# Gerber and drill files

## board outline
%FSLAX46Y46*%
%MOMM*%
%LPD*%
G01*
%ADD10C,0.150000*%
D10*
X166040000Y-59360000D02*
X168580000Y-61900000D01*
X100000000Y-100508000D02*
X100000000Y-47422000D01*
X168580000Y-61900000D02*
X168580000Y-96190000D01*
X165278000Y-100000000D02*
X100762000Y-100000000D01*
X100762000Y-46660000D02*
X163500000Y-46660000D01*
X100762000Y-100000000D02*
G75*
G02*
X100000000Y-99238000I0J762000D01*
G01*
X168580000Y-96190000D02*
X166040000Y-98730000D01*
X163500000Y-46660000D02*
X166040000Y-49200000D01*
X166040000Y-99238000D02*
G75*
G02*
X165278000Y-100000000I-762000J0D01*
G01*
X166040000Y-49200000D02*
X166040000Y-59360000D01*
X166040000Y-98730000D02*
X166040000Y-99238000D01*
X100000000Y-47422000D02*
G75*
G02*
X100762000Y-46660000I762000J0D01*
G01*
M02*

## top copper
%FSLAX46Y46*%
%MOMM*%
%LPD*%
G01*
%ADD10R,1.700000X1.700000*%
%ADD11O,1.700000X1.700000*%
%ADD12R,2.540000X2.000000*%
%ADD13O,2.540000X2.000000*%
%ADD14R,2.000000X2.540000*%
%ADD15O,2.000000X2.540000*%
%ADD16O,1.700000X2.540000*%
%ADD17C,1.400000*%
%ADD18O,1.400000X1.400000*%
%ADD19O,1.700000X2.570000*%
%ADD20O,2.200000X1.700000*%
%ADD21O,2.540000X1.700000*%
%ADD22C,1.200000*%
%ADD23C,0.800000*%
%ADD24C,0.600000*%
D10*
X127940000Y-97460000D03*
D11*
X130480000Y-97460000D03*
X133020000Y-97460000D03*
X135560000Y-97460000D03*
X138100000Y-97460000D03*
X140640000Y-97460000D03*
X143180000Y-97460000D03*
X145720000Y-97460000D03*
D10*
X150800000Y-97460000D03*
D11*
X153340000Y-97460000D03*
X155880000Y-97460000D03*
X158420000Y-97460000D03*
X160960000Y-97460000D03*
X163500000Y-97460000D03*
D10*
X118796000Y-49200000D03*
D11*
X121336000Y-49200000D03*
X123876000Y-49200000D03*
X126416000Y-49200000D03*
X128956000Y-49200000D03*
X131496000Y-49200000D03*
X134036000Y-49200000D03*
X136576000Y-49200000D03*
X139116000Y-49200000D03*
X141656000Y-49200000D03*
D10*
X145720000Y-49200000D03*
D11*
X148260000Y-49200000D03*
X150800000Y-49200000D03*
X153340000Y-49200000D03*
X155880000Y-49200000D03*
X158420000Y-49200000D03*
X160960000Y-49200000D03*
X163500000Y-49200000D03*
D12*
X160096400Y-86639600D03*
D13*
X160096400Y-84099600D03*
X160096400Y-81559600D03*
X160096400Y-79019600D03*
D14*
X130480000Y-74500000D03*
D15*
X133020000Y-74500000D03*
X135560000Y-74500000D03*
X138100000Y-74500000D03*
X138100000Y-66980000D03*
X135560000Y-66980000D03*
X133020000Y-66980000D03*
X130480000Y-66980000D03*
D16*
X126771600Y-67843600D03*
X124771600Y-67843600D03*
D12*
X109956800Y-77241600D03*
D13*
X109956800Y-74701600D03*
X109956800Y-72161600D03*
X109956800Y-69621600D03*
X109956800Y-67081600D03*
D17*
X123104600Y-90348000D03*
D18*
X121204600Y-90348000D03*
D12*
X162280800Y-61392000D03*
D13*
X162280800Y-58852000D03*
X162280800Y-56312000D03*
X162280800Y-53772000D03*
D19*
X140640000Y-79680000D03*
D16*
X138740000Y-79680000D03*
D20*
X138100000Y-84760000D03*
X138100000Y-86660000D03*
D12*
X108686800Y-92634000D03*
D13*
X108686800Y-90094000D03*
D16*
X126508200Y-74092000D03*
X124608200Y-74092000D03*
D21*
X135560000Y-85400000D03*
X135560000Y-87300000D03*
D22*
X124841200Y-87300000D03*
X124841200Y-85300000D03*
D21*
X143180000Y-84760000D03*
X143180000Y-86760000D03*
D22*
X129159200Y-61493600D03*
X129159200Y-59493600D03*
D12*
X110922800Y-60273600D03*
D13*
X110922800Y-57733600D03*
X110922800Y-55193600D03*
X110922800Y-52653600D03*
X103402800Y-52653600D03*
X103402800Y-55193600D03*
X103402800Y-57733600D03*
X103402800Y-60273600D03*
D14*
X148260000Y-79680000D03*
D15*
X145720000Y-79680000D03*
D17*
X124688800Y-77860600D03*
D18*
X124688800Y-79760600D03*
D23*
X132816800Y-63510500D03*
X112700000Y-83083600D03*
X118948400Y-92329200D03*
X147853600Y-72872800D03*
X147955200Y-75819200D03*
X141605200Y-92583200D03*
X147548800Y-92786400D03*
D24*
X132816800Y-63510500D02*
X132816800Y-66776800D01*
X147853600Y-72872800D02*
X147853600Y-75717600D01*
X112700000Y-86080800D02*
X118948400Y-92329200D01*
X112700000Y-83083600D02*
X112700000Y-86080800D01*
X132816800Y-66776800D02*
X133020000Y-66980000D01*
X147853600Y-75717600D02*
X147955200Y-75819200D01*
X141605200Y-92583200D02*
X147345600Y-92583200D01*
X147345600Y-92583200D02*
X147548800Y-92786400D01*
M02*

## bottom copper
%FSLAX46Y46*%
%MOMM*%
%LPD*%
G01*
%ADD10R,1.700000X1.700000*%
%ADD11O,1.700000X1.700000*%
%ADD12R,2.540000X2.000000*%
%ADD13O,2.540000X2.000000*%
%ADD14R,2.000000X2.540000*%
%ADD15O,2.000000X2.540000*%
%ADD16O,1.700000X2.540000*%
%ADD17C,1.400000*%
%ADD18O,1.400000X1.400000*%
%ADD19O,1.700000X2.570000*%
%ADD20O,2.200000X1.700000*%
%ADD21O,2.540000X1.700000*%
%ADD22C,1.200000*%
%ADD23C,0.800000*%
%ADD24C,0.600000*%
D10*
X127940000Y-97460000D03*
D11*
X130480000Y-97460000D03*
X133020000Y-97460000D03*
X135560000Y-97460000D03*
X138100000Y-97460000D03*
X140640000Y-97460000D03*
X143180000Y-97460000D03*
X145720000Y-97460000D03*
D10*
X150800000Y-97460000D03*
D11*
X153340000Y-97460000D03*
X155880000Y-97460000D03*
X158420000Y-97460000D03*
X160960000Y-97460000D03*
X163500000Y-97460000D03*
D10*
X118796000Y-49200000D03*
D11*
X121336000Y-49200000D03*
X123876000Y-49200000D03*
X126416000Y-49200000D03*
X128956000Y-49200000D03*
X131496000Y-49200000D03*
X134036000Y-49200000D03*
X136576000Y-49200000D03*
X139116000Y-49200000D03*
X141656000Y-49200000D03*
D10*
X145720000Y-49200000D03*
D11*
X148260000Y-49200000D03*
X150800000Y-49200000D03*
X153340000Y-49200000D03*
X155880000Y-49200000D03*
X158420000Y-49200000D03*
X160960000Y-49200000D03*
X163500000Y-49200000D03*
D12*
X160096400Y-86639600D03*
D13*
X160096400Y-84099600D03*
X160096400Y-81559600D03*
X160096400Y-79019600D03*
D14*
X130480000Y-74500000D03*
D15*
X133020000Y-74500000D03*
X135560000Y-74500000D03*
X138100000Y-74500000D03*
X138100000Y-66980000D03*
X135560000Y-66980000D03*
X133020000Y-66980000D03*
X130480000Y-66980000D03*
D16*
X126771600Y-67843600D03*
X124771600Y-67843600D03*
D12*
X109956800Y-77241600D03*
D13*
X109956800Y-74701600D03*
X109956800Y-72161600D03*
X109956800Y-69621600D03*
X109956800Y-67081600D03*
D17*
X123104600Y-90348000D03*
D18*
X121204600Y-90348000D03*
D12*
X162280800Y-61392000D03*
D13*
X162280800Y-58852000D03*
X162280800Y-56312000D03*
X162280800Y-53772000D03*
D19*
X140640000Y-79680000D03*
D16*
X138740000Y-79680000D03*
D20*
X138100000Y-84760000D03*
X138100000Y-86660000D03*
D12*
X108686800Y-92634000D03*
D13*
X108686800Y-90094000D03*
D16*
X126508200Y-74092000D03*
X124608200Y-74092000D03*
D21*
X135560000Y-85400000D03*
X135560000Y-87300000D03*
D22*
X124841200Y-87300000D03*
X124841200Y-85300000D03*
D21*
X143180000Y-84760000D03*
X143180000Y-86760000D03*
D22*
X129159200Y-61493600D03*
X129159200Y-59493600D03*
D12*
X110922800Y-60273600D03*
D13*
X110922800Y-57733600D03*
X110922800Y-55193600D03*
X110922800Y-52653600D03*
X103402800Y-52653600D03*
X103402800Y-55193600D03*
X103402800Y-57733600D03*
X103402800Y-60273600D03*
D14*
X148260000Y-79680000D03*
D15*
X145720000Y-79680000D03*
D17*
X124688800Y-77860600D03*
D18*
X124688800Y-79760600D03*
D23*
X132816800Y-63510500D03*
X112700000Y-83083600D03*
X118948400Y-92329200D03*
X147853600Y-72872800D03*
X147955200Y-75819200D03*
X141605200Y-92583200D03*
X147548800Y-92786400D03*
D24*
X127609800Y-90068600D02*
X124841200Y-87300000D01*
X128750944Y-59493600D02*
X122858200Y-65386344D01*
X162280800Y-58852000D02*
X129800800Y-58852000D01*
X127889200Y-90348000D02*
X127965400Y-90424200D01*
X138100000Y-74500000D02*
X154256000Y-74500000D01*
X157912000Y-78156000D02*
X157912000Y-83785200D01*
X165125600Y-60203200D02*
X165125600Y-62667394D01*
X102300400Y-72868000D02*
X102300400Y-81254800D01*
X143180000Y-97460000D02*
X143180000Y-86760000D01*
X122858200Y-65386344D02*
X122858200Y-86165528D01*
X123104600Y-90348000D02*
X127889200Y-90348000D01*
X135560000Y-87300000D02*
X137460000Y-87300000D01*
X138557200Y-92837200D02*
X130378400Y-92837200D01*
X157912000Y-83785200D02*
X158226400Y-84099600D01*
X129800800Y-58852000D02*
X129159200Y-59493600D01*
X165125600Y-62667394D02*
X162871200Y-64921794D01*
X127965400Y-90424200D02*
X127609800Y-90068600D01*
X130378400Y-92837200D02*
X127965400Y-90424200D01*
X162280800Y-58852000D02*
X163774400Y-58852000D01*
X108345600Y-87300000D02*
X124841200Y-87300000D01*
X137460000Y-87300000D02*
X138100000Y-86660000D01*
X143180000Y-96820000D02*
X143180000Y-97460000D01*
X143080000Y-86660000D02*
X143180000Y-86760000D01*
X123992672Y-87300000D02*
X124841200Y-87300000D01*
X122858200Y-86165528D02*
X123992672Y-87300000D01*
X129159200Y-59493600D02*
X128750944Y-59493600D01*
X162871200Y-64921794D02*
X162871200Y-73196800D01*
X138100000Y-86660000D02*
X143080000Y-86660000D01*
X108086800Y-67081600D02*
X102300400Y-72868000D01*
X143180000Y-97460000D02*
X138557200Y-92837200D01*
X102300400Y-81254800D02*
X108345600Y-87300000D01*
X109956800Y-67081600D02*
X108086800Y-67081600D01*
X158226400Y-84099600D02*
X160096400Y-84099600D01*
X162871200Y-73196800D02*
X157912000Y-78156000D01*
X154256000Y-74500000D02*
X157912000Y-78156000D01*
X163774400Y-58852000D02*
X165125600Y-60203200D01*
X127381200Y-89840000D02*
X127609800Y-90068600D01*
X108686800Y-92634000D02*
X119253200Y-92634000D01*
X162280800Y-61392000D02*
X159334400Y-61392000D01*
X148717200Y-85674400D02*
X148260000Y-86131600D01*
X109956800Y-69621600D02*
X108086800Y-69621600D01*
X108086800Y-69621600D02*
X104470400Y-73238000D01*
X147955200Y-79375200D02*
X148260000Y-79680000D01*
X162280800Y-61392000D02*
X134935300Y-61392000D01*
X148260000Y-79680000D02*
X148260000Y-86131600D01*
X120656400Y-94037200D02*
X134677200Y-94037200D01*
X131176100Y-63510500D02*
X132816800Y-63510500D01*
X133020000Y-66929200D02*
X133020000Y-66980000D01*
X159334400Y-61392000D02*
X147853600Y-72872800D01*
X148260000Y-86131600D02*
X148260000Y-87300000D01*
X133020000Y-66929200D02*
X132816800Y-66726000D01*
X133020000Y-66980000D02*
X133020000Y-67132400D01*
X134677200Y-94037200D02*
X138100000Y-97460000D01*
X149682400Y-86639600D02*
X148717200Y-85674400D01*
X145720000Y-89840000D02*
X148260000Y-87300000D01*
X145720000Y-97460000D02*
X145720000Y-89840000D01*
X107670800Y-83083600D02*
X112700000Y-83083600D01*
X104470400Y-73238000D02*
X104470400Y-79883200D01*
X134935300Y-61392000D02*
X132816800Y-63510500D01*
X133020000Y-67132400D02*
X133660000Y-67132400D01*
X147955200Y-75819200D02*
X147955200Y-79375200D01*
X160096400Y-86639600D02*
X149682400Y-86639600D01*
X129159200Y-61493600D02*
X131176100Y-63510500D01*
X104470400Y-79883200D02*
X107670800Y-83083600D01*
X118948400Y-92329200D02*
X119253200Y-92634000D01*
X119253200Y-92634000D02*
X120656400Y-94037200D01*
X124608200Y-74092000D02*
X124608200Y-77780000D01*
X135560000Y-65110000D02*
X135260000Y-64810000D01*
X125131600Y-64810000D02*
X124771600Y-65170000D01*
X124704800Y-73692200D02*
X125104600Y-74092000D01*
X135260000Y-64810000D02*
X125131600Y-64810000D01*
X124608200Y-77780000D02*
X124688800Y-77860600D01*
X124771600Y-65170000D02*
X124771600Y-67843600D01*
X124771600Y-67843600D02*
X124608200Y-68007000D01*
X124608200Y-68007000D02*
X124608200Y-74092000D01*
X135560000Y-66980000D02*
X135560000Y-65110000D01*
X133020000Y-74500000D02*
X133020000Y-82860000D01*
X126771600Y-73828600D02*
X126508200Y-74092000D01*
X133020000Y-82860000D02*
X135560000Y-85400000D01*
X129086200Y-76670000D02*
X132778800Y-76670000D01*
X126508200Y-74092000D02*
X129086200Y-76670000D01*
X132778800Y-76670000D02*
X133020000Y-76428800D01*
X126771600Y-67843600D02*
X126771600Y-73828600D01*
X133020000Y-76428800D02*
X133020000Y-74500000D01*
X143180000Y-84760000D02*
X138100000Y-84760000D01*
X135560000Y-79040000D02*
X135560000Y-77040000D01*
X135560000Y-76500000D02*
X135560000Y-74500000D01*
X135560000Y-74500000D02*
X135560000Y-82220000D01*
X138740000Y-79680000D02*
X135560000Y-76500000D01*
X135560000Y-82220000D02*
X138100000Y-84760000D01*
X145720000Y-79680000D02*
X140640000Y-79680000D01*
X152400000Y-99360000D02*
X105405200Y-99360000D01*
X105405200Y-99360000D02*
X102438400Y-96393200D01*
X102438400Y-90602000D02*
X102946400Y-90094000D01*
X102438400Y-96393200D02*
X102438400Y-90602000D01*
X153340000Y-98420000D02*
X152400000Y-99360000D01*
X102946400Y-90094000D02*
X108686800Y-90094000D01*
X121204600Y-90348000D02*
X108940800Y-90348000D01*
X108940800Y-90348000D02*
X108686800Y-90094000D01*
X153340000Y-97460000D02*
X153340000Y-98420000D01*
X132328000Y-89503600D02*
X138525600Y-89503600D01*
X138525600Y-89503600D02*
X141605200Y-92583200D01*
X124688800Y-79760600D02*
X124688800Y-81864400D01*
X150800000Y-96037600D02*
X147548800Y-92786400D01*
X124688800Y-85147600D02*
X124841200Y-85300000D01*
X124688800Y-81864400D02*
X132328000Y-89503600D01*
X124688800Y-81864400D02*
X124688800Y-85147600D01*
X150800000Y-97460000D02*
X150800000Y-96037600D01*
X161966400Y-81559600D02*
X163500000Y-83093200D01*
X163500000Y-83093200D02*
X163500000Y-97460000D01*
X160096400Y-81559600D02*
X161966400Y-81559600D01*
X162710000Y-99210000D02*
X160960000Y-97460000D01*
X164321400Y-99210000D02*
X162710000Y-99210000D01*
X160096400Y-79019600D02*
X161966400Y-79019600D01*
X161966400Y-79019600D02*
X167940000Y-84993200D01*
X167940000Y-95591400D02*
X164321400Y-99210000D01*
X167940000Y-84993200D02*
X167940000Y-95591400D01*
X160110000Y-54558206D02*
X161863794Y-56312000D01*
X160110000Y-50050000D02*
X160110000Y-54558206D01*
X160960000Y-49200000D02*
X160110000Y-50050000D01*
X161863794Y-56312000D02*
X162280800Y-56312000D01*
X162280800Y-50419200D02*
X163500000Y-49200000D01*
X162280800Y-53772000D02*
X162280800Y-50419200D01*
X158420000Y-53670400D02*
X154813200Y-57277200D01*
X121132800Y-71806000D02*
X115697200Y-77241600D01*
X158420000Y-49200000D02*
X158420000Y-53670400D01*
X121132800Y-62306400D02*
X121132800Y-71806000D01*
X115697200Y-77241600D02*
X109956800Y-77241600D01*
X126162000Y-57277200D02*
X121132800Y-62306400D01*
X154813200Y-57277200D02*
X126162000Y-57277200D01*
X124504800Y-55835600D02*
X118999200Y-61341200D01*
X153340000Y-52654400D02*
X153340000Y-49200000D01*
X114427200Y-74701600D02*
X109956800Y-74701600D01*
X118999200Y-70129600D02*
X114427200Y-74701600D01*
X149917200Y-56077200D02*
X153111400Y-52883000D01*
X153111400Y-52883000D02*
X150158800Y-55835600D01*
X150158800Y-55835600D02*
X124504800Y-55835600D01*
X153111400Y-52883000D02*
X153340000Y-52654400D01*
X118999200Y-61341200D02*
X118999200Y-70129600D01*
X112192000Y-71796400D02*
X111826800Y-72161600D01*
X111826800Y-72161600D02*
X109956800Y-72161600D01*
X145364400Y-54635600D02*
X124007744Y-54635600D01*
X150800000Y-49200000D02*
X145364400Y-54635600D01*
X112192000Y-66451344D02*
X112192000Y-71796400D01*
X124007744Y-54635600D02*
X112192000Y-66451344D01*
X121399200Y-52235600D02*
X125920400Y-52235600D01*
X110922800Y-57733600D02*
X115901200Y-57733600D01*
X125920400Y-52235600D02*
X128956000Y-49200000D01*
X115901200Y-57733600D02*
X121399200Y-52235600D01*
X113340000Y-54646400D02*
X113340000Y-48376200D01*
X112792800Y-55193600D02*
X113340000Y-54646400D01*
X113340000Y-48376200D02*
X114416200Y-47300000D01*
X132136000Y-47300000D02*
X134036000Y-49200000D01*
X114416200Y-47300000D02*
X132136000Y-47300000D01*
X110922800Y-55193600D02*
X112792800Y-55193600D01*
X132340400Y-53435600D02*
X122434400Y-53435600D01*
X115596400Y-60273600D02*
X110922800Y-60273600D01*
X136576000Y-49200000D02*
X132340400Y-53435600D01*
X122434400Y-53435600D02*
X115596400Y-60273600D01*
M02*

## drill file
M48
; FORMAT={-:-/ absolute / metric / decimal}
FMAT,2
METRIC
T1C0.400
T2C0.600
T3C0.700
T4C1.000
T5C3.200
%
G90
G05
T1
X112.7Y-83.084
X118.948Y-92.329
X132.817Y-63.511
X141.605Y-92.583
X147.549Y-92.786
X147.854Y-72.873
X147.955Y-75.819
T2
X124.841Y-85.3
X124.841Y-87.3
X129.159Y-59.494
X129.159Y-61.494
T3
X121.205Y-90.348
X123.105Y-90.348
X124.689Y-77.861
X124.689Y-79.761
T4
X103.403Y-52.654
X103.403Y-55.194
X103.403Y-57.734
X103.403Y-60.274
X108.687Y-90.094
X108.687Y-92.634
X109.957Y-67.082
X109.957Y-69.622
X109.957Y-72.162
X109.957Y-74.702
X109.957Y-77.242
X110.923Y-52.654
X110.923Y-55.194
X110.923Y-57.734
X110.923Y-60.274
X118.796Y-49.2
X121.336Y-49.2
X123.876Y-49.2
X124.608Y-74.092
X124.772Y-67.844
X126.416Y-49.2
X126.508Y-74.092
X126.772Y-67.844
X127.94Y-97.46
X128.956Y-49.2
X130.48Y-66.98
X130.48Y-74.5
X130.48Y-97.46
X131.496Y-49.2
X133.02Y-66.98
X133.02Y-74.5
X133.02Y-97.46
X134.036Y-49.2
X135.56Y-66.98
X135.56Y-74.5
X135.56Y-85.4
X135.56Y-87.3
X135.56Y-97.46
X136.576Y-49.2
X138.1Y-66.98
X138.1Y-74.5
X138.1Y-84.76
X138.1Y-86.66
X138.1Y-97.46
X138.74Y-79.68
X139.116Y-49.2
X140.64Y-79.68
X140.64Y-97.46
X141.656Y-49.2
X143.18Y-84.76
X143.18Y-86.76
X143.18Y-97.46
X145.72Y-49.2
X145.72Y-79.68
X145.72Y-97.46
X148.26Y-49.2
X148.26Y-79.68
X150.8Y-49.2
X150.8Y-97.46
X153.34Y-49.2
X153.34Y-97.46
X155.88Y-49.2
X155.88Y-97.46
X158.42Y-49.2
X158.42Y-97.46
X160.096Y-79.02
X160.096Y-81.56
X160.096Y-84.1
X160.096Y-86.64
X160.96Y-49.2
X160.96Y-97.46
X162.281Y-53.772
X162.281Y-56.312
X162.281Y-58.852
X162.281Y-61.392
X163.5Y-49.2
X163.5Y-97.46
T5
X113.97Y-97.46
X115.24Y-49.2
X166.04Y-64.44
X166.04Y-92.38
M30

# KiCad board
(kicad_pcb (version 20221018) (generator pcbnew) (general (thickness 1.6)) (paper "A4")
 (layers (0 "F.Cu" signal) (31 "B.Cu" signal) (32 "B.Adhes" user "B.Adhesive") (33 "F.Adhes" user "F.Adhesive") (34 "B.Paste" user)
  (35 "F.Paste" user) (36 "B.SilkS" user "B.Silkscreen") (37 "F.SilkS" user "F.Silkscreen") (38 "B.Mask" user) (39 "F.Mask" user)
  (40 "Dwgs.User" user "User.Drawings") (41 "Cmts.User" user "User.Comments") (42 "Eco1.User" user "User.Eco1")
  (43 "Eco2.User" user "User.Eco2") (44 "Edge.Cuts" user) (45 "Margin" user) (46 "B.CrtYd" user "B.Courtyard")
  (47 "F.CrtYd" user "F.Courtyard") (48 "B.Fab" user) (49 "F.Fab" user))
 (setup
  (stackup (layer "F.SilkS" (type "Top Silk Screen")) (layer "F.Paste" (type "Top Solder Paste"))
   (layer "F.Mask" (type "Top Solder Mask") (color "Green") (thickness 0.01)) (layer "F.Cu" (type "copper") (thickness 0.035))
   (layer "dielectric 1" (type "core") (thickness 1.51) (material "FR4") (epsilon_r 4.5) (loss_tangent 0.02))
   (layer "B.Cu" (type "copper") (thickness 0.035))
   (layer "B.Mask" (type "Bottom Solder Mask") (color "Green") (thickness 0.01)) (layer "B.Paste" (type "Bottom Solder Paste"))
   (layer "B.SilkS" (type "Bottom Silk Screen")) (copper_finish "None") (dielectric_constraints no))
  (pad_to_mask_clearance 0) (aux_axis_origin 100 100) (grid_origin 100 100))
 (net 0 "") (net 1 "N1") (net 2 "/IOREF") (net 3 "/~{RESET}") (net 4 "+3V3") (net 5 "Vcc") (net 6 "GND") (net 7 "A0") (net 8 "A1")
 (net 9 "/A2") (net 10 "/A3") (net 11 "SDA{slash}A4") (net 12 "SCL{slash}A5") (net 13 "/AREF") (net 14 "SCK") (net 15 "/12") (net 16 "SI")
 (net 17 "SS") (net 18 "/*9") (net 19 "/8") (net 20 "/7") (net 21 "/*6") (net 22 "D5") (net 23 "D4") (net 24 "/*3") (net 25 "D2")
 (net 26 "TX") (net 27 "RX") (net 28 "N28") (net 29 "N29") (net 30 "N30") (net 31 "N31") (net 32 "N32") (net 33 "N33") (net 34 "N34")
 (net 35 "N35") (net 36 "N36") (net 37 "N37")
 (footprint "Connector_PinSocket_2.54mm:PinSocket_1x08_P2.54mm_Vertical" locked (layer "F.Cu") (at 127.94 97.46 90)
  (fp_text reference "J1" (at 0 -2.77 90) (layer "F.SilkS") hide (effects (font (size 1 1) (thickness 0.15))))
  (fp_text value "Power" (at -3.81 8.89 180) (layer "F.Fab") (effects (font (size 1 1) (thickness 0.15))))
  (pad "1" thru_hole rect locked (at 0 0 90) (size 1.7 1.7) (drill 1) (layers "*.Cu" "*.Mask") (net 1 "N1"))
  (pad "2" thru_hole oval locked (at 0 2.54 90) (size 1.7 1.7) (drill 1) (layers "*.Cu" "*.Mask") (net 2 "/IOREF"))
  (pad "3" thru_hole oval locked (at 0 5.08 90) (size 1.7 1.7) (drill 1) (layers "*.Cu" "*.Mask") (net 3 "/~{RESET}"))
  (pad "4" thru_hole oval locked (at 0 7.62 90) (size 1.7 1.7) (drill 1) (layers "*.Cu" "*.Mask") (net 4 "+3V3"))
  (pad "5" thru_hole oval locked (at 0 10.16 90) (size 1.7 1.7) (drill 1) (layers "*.Cu" "*.Mask") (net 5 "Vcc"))
  (pad "6" thru_hole oval locked (at 0 12.7 90) (size 1.7 1.7) (drill 1) (layers "*.Cu" "*.Mask") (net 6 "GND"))
  (pad "7" thru_hole oval locked (at 0 15.24 90) (size 1.7 1.7) (drill 1) (layers "*.Cu" "*.Mask") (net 6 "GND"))
  (pad "8" thru_hole oval locked (at 0 17.78 90) (size 1.7 1.7) (drill 1) (layers "*.Cu" "*.Mask") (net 5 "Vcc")))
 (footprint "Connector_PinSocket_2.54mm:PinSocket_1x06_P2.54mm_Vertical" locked (layer "F.Cu") (at 150.8 97.46 90)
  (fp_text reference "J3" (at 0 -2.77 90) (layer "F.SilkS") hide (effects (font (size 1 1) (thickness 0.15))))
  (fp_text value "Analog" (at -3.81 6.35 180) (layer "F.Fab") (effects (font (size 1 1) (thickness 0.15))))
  (pad "1" thru_hole rect locked (at 0 0 90) (size 1.7 1.7) (drill 1) (layers "*.Cu" "*.Mask") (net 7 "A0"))
  (pad "2" thru_hole oval locked (at 0 2.54 90) (size 1.7 1.7) (drill 1) (layers "*.Cu" "*.Mask") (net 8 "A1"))
  (pad "3" thru_hole oval locked (at 0 5.08 90) (size 1.7 1.7) (drill 1) (layers "*.Cu" "*.Mask") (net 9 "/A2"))
  (pad "4" thru_hole oval locked (at 0 7.62 90) (size 1.7 1.7) (drill 1) (layers "*.Cu" "*.Mask") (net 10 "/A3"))
  (pad "5" thru_hole oval locked (at 0 10.16 90) (size 1.7 1.7) (drill 1) (layers "*.Cu" "*.Mask") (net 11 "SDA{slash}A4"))
  (pad "6" thru_hole oval locked (at 0 12.7 90) (size 1.7 1.7) (drill 1) (layers "*.Cu" "*.Mask") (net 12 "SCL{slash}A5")))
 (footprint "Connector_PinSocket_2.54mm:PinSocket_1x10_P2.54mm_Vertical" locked (layer "F.Cu") (at 118.796 49.2 90)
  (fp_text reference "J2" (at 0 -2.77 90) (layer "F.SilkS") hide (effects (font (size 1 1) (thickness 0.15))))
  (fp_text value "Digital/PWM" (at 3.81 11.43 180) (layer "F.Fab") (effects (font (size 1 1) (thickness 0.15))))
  (pad "1" thru_hole rect locked (at 0 0 90) (size 1.7 1.7) (drill 1) (layers "*.Cu" "*.Mask") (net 12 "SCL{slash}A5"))
  (pad "2" thru_hole oval locked (at 0 2.54 90) (size 1.7 1.7) (drill 1) (layers "*.Cu" "*.Mask") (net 11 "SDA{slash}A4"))
  (pad "3" thru_hole oval locked (at 0 5.08 90) (size 1.7 1.7) (drill 1) (layers "*.Cu" "*.Mask") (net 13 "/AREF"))
  (pad "4" thru_hole oval locked (at 0 7.62 90) (size 1.7 1.7) (drill 1) (layers "*.Cu" "*.Mask") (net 6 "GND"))
  (pad "5" thru_hole oval locked (at 0 10.16 90) (size 1.7 1.7) (drill 1) (layers "*.Cu" "*.Mask") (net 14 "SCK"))
  (pad "6" thru_hole oval locked (at 0 12.7 90) (size 1.7 1.7) (drill 1) (layers "*.Cu" "*.Mask") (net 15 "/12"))
  (pad "7" thru_hole oval locked (at 0 15.24 90) (size 1.7 1.7) (drill 1) (layers "*.Cu" "*.Mask") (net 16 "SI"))
  (pad "8" thru_hole oval locked (at 0 17.78 90) (size 1.7 1.7) (drill 1) (layers "*.Cu" "*.Mask") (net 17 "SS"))
  (pad "9" thru_hole oval locked (at 0 20.32 90) (size 1.7 1.7) (drill 1) (layers "*.Cu" "*.Mask") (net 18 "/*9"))
  (pad "10" thru_hole oval locked (at 0 22.86 90) (size 1.7 1.7) (drill 1) (layers "*.Cu" "*.Mask") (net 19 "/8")))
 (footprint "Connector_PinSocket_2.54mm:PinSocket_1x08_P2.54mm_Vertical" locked (layer "F.Cu") (at 145.72 49.2 90)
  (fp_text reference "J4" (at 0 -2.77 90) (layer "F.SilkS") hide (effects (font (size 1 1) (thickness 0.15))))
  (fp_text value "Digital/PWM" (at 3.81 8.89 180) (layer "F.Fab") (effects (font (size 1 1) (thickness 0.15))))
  (pad "1" thru_hole rect locked (at 0 0 90) (size 1.7 1.7) (drill 1) (layers "*.Cu" "*.Mask") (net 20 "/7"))
  (pad "2" thru_hole oval locked (at 0 2.54 90) (size 1.7 1.7) (drill 1) (layers "*.Cu" "*.Mask") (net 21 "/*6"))
  (pad "3" thru_hole oval locked (at 0 5.08 90) (size 1.7 1.7) (drill 1) (layers "*.Cu" "*.Mask") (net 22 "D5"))
  (pad "4" thru_hole oval locked (at 0 7.62 90) (size 1.7 1.7) (drill 1) (layers "*.Cu" "*.Mask") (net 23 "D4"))
  (pad "5" thru_hole oval locked (at 0 10.16 90) (size 1.7 1.7) (drill 1) (layers "*.Cu" "*.Mask") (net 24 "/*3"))
  (pad "6" thru_hole oval locked (at 0 12.7 90) (size 1.7 1.7) (drill 1) (layers "*.Cu" "*.Mask") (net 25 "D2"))
  (pad "7" thru_hole oval locked (at 0 15.24 90) (size 1.7 1.7) (drill 1) (layers "*.Cu" "*.Mask") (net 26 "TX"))
  (pad "8" thru_hole oval locked (at 0 17.78 90) (size 1.7 1.7) (drill 1) (layers "*.Cu" "*.Mask") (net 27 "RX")))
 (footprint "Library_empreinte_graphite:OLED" (layer "F.Cu") (at 160.0964 82.8296 90)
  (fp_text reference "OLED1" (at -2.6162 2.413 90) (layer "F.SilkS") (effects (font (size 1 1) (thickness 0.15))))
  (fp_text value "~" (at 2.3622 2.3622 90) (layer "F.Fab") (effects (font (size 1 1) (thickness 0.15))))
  (pad "1" thru_hole rect (at -3.81 0 90) (size 2 2.54) (drill 1) (layers "*.Cu" "*.Mask") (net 5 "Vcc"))
  (pad "2" thru_hole oval (at -1.27 0 90) (size 2 2.54) (drill 1) (layers "*.Cu" "*.Mask") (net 6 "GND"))
  (pad "3" thru_hole oval (at 1.27 0 90) (size 2 2.54) (drill 1) (layers "*.Cu" "*.Mask") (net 12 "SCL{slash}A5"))
  (pad "4" thru_hole oval (at 3.81 0 90) (size 2 2.54) (drill 1) (layers "*.Cu" "*.Mask") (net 11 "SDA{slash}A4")))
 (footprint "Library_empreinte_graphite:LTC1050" (layer "F.Cu") (at 134.29 70.74)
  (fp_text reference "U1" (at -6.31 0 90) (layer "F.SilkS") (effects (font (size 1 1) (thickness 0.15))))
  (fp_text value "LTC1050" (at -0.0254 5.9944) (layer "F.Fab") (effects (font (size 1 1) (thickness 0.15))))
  (pad "1" thru_hole rect (at -3.81 3.76) (size 2 2.54) (drill 1) (layers "*.Cu" "*.Mask") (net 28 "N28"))
  (pad "2" thru_hole oval (at -1.27 3.76) (size 2 2.54) (drill 1) (layers "*.Cu" "*.Mask") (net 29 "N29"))
  (pad "3" thru_hole oval (at 1.27 3.76) (size 2 2.54) (drill 1) (layers "*.Cu" "*.Mask") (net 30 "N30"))
  (pad "4" thru_hole oval (at 3.81 3.76) (size 2 2.54) (drill 1) (layers "*.Cu" "*.Mask") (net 6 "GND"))
  (pad "5" thru_hole oval (at 3.81 -3.76) (size 2 2.54) (drill 1) (layers "*.Cu" "*.Mask") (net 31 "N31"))
  (pad "6" thru_hole oval (at 1.27 -3.76) (size 2 2.54) (drill 1) (layers "*.Cu" "*.Mask") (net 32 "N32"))
  (pad "7" thru_hole oval (at -1.27 -3.76) (size 2 2.54) (drill 1) (layers "*.Cu" "*.Mask") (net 5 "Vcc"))
  (pad "8" thru_hole oval (at -3.81 -3.76) (size 2 2.54) (drill 1) (layers "*.Cu" "*.Mask") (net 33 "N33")))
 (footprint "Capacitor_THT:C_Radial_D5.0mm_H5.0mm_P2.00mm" (layer "F.Cu") (at 126.7716 67.8436 180)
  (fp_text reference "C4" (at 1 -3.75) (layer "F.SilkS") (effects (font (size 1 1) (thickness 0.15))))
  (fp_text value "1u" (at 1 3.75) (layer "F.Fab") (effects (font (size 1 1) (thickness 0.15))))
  (pad "1" thru_hole oval (at 0 0 180) (size 1.7 2.54) (drill 1) (layers "*.Cu" "*.Mask") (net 29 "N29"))
  (pad "2" thru_hole oval (at 2 0 180) (size 1.7 2.54) (drill 1) (layers "*.Cu" "*.Mask") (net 32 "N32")))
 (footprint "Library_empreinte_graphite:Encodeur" (layer "F.Cu") (at 109.9568 72.1616 90)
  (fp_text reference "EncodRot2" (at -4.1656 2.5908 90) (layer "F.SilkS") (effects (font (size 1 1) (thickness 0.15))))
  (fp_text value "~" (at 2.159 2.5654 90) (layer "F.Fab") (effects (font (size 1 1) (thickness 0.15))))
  (pad "1" thru_hole rect (at -5.08 0 90) (size 2 2.54) (drill 1) (layers "*.Cu" "*.Mask") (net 25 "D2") (thermal_bridge_angle 45))
  (pad "2" thru_hole oval (at -2.54 0 90) (size 2 2.54) (drill 1) (layers "*.Cu" "*.Mask") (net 23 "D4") (thermal_bridge_angle 45))
  (pad "3" thru_hole oval (at 0 0 90) (size 2 2.54) (drill 1) (layers "*.Cu" "*.Mask") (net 22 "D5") (thermal_bridge_angle 45))
  (pad "4" thru_hole oval (at 2.54 0 90) (size 2 2.54) (drill 1) (layers "*.Cu" "*.Mask") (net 5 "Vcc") (thermal_bridge_angle 45))
  (pad "5" thru_hole oval (at 5.08 0 90) (size 2 2.54) (drill 1) (layers "*.Cu" "*.Mask") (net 6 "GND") (thermal_bridge_angle 45)))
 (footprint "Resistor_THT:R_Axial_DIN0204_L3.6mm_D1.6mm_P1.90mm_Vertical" (layer "F.Cu") (at 123.1046 90.348 180)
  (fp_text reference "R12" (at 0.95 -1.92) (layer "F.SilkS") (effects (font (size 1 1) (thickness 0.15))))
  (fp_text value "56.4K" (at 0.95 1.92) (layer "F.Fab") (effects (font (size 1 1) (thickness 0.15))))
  (pad "1" thru_hole circle (at 0 0 180) (size 1.4 1.4) (drill 0.7) (layers "*.Cu" "*.Mask") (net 6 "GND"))
  (pad "2" thru_hole oval (at 1.9 0 180) (size 1.4 1.4) (drill 0.7) (layers "*.Cu" "*.Mask") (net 8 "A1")))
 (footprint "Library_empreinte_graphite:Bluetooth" (layer "F.Cu") (at 162.2808 57.582 90)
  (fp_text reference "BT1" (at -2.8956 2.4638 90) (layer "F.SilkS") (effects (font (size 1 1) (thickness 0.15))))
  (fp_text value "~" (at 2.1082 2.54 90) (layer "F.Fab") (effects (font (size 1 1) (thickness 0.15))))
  (pad "1" thru_hole rect (at -3.81 0 90) (size 2 2.54) (drill 1) (layers "*.Cu" "*.Mask") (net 5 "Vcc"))
  (pad "2" thru_hole oval (at -1.27 0 90) (size 2 2.54) (drill 1) (layers "*.Cu" "*.Mask") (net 6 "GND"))
  (pad "3" thru_hole oval (at 1.27 0 90) (size 2 2.54) (drill 1) (layers "*.Cu" "*.Mask") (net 26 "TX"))
  (pad "4" thru_hole oval (at 3.81 0 90) (size 2 2.54) (drill 1) (layers "*.Cu" "*.Mask") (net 27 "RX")))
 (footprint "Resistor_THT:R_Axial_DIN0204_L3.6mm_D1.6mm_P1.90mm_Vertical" (layer "F.Cu") (at 140.64 79.68 180)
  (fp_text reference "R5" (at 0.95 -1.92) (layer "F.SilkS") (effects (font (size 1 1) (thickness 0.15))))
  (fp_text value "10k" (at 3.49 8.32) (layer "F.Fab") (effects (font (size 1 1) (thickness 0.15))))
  (pad "1" thru_hole oval (at 0 0 180) (size 1.7 2.57) (drill 1) (layers "*.Cu" "*.Mask") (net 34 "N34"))
  (pad "2" thru_hole oval (at 1.9 0 180) (size 1.7 2.54) (drill 1) (layers "*.Cu" "*.Mask") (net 30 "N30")))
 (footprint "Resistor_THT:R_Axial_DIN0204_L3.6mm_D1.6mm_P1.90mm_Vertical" (layer "F.Cu") (at 138.1 84.76 -90)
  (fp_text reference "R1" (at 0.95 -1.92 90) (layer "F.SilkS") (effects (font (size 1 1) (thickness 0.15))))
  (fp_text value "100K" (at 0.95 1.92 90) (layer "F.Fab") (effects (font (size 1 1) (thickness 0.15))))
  (pad "1" thru_hole oval (at 0 0 270) (size 1.7 2.2) (drill 1) (layers "*.Cu" "*.Mask") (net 30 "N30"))
  (pad "2" thru_hole oval (at 1.9 0 270) (size 1.7 2.2) (drill 1) (layers "*.Cu" "*.Mask") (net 6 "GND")))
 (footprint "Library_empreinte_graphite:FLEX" (layer "F.Cu") (at 108.6868 91.364 90)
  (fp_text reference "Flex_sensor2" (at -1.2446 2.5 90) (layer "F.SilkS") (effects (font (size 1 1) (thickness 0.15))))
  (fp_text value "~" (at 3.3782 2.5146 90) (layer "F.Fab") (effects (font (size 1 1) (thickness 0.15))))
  (pad "1" thru_hole rect (at -1.27 0 90) (size 2 2.54) (drill 1) (layers "*.Cu" "*.Mask") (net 5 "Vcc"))
  (pad "2" thru_hole oval (at 1.27 0 90) (size 2 2.54) (drill 1) (layers "*.Cu" "*.Mask") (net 8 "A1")))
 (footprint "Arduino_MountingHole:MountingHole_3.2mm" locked (layer "F.Cu") (at 115.24 49.2)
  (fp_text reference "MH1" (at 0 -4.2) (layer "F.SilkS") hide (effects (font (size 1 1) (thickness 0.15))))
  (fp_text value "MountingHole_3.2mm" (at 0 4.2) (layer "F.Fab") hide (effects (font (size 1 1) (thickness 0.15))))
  (pad "" np_thru_hole circle locked (at 0 0) (size 3.2 3.2) (drill 3.2) (layers "*.Cu" "*.Mask")))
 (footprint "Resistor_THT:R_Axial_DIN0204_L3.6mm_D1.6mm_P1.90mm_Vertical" (layer "F.Cu") (at 126.5082 74.092 180)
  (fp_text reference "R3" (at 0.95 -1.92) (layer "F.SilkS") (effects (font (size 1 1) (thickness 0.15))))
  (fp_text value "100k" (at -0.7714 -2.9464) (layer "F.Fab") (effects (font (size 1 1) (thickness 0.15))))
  (pad "1" thru_hole oval (at 0 0 180) (size 1.7 2.54) (drill 1) (layers "*.Cu" "*.Mask") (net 29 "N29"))
  (pad "2" thru_hole oval (at 1.9 0 180) (size 1.7 2.54) (drill 1) (layers "*.Cu" "*.Mask") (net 32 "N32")))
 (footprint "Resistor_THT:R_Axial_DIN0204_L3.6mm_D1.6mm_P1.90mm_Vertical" (layer "F.Cu") (at 135.56 85.4 -90)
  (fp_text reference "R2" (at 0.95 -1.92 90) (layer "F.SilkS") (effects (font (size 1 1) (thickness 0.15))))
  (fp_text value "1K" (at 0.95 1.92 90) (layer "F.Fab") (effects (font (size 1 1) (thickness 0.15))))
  (pad "1" thru_hole oval (at 0 0 270) (size 1.7 2.54) (drill 1) (layers "*.Cu" "*.Mask") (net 29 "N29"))
  (pad "2" thru_hole oval (at 1.9 0 270) (size 1.7 2.54) (drill 1) (layers "*.Cu" "*.Mask") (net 6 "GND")))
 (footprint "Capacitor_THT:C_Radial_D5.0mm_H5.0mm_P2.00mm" (layer "F.Cu") (at 124.8412 87.3 90)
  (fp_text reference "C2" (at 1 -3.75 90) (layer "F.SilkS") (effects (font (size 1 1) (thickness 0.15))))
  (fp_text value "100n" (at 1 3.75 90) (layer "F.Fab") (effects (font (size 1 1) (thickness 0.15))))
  (pad "1" thru_hole circle (at 0 0 90) (size 1.2 1.2) (drill 0.6) (layers "*.Cu" "*.Mask") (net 6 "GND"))
  (pad "2" thru_hole circle (at 2 0 90) (size 1.2 1.2) (drill 0.6) (layers "*.Cu" "*.Mask") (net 7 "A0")))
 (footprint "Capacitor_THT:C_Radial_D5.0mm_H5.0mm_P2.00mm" (layer "F.Cu") (at 143.18 84.76 -90)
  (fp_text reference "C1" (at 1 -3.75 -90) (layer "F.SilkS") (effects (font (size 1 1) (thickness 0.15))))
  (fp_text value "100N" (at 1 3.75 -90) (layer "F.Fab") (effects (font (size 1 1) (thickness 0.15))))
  (pad "1" thru_hole oval (at 0 0 270) (size 1.7 2.54) (drill 1) (layers "*.Cu" "*.Mask") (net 30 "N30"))
  (pad "2" thru_hole oval (at 2 0 270) (size 1.7 2.54) (drill 1) (layers "*.Cu" "*.Mask") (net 6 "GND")))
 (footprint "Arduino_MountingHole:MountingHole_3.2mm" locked (layer "F.Cu") (at 113.97 97.46)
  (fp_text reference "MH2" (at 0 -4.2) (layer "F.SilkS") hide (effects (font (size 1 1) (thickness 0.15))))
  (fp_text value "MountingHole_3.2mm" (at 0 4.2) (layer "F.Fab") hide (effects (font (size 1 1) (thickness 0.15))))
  (pad "" np_thru_hole circle locked (at 0 0) (size 3.2 3.2) (drill 3.2) (layers "*.Cu" "*.Mask")))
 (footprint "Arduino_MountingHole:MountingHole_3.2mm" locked (layer "F.Cu") (at 166.04 64.44)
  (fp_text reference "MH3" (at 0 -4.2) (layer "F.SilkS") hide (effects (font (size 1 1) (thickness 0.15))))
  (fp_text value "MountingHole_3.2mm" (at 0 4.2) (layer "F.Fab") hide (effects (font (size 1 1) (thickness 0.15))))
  (pad "" np_thru_hole circle locked (at 0 0) (size 3.2 3.2) (drill 3.2) (layers "*.Cu" "*.Mask")))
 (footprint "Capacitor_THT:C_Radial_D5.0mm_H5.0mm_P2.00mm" (layer "F.Cu") (at 129.1592 61.4936 90)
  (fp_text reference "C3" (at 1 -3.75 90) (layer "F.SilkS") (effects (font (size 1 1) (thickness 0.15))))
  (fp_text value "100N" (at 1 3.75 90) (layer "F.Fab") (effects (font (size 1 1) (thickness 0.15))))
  (pad "1" thru_hole circle (at 0 0 90) (size 1.2 1.2) (drill 0.6) (layers "*.Cu" "*.Mask") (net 5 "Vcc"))
  (pad "2" thru_hole circle (at 2 0 90) (size 1.2 1.2) (drill 0.6) (layers "*.Cu" "*.Mask") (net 6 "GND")))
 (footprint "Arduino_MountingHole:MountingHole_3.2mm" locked (layer "F.Cu") (at 166.04 92.38)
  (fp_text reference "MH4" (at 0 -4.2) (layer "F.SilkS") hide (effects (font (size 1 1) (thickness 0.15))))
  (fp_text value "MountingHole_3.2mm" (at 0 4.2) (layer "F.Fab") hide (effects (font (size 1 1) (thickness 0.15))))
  (pad "" np_thru_hole circle locked (at 0 0) (size 3.2 3.2) (drill 3.2) (layers "*.Cu" "*.Mask")))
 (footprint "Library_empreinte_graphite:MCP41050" (layer "F.Cu") (at 107.1628 56.4636 90)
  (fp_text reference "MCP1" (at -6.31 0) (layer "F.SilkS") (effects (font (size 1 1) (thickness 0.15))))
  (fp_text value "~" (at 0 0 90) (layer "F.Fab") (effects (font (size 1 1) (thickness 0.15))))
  (pad "1" thru_hole rect (at -3.81 3.76 90) (size 2 2.54) (drill 1) (layers "*.Cu" "*.Mask") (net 17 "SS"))
  (pad "2" thru_hole oval (at -1.27 3.76 90) (size 2 2.54) (drill 1) (layers "*.Cu" "*.Mask") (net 14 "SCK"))
  (pad "3" thru_hole oval (at 1.27 3.76 90) (size 2 2.54) (drill 1) (layers "*.Cu" "*.Mask") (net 16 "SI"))
  (pad "4" thru_hole oval (at 3.81 3.76 90) (size 2 2.54) (drill 1) (layers "*.Cu" "*.Mask") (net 6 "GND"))
  (pad "5" thru_hole oval (at 3.81 -3.76 90) (size 2 2.54) (drill 1) (layers "*.Cu" "*.Mask") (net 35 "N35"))
  (pad "6" thru_hole oval (at 1.27 -3.76 90) (size 2 2.54) (drill 1) (layers "*.Cu" "*.Mask") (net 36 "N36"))
  (pad "7" thru_hole oval (at -1.27 -3.76 90) (size 2 2.54) (drill 1) (layers "*.Cu" "*.Mask") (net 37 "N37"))
  (pad "8" thru_hole oval (at -3.81 -3.76 90) (size 2 2.54) (drill 1) (layers "*.Cu" "*.Mask") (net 5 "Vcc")))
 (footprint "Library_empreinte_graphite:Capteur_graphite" (layer "F.Cu") (at 146.99 79.68 180)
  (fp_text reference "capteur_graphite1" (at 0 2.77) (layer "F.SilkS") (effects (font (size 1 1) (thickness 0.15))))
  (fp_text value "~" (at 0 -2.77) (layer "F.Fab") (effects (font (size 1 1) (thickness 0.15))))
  (pad "1" thru_hole rect (at -1.27 0 180) (size 2 2.54) (drill 1) (layers "*.Cu" "*.Mask") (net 5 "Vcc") (thermal_bridge_angle 45))
  (pad "2" thru_hole oval (at 1.27 0 180) (size 2 2.54) (drill 1) (layers "*.Cu" "*.Mask") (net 34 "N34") (thermal_bridge_angle 45)))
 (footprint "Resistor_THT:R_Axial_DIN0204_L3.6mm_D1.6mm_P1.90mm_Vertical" (layer "F.Cu") (at 124.6888 77.8606 -90)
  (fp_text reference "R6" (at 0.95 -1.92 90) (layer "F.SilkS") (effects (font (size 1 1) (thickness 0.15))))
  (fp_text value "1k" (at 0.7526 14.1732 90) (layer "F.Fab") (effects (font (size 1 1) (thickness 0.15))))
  (pad "1" thru_hole circle (at 0 0 270) (size 1.4 1.4) (drill 0.7) (layers "*.Cu" "*.Mask") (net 32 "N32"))
  (pad "2" thru_hole oval (at 1.9 0 270) (size 1.4 1.4) (drill 0.7) (layers "*.Cu" "*.Mask") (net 7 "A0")))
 (gr_line (start 166.04 59.36) (end 168.58 61.9) (stroke (width 0.15) (type solid)) (layer "Edge.Cuts"))
 (gr_line (start 100 100.508) (end 100 47.422) (stroke (width 0.15) (type solid)) (layer "Edge.Cuts"))
 (gr_line (start 168.58 61.9) (end 168.58 96.19) (stroke (width 0.15) (type solid)) (layer "Edge.Cuts"))
 (gr_line (start 165.278 100) (end 100.762 100) (stroke (width 0.15) (type solid)) (layer "Edge.Cuts"))
 (gr_line (start 100.762 46.66) (end 163.5 46.66) (stroke (width 0.15) (type solid)) (layer "Edge.Cuts"))
 (gr_arc (start 100.762 100) (mid 100.223185 99.776815) (end 100 99.238) (stroke (width 0.15) (type solid)) (layer "Edge.Cuts"))
 (gr_line (start 168.58 96.19) (end 166.04 98.73) (stroke (width 0.15) (type solid)) (layer "Edge.Cuts"))
 (gr_line (start 163.5 46.66) (end 166.04 49.2) (stroke (width 0.15) (type solid)) (layer "Edge.Cuts"))
 (gr_arc (start 166.04 99.238) (mid 165.816815 99.776815) (end 165.278 100) (stroke (width 0.15) (type solid)) (layer "Edge.Cuts"))
 (gr_line (start 166.04 49.2) (end 166.04 59.36) (stroke (width 0.15) (type solid)) (layer "Edge.Cuts"))
 (gr_line (start 166.04 98.73) (end 166.04 99.238) (stroke (width 0.15) (type solid)) (layer "Edge.Cuts"))
 (gr_arc (start 100 47.422) (mid 100.223185 46.883185) (end 100.762 46.66) (stroke (width 0.15) (type solid)) (layer "Edge.Cuts"))
 (segment (start 127.6098 90.0686) (end 124.8412 87.3) (width 0.6) (layer "B.Cu") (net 6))
 (segment (start 128.750944 59.4936) (end 122.8582 65.386344) (width 0.6) (layer "B.Cu") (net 6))
 (segment (start 162.2808 58.852) (end 129.8008 58.852) (width 0.6) (layer "B.Cu") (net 6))
 (segment (start 127.8892 90.348) (end 127.9654 90.4242) (width 0.6) (layer "B.Cu") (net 6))
 (segment (start 138.1 74.5) (end 154.256 74.5) (width 0.6) (layer "B.Cu") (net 6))
 (segment (start 157.912 78.156) (end 157.912 83.7852) (width 0.6) (layer "B.Cu") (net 6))
 (segment (start 165.1256 60.2032) (end 165.1256 62.667394) (width 0.6) (layer "B.Cu") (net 6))
 (segment (start 102.3004 72.868) (end 102.3004 81.2548) (width 0.6) (layer "B.Cu") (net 6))
 (segment (start 143.18 97.46) (end 143.18 86.76) (width 0.6) (layer "B.Cu") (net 6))
 (segment (start 122.8582 65.386344) (end 122.8582 86.165528) (width 0.6) (layer "B.Cu") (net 6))
 (segment (start 123.1046 90.348) (end 127.8892 90.348) (width 0.6) (layer "B.Cu") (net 6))
 (segment (start 135.56 87.3) (end 137.46 87.3) (width 0.6) (layer "B.Cu") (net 6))
 (segment (start 138.5572 92.8372) (end 130.3784 92.8372) (width 0.6) (layer "B.Cu") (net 6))
 (segment (start 157.912 83.7852) (end 158.2264 84.0996) (width 0.6) (layer "B.Cu") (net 6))
 (segment (start 129.8008 58.852) (end 129.1592 59.4936) (width 0.6) (layer "B.Cu") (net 6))
 (segment (start 165.1256 62.667394) (end 162.8712 64.921794) (width 0.6) (layer "B.Cu") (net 6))
 (segment (start 127.9654 90.4242) (end 127.6098 90.0686) (width 0.6) (layer "B.Cu") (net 6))
 (segment (start 130.3784 92.8372) (end 127.9654 90.4242) (width 0.6) (layer "B.Cu") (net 6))
 (segment (start 162.2808 58.852) (end 163.7744 58.852) (width 0.6) (layer "B.Cu") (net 6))
 (segment (start 108.3456 87.3) (end 124.8412 87.3) (width 0.6) (layer "B.Cu") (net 6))
 (segment (start 137.46 87.3) (end 138.1 86.66) (width 0.6) (layer "B.Cu") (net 6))
 (segment (start 143.18 96.82) (end 143.18 97.46) (width 0.6) (layer "B.Cu") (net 6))
 (segment (start 143.08 86.66) (end 143.18 86.76) (width 0.6) (layer "B.Cu") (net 6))
 (segment (start 123.992672 87.3) (end 124.8412 87.3) (width 0.6) (layer "B.Cu") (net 6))
 (segment (start 122.8582 86.165528) (end 123.992672 87.3) (width 0.6) (layer "B.Cu") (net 6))
 (segment (start 129.1592 59.4936) (end 128.750944 59.4936) (width 0.6) (layer "B.Cu") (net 6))
 (segment (start 162.8712 64.921794) (end 162.8712 73.1968) (width 0.6) (layer "B.Cu") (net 6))
 (segment (start 138.1 86.66) (end 143.08 86.66) (width 0.6) (layer "B.Cu") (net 6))
 (segment (start 108.0868 67.0816) (end 102.3004 72.868) (width 0.6) (layer "B.Cu") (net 6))
 (segment (start 143.18 97.46) (end 138.5572 92.8372) (width 0.6) (layer "B.Cu") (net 6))
 (segment (start 102.3004 81.2548) (end 108.3456 87.3) (width 0.6) (layer "B.Cu") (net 6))
 (segment (start 109.9568 67.0816) (end 108.0868 67.0816) (width 0.6) (layer "B.Cu") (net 6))
 (segment (start 158.2264 84.0996) (end 160.0964 84.0996) (width 0.6) (layer "B.Cu") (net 6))
 (segment (start 162.8712 73.1968) (end 157.912 78.156) (width 0.6) (layer "B.Cu") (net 6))
 (segment (start 154.256 74.5) (end 157.912 78.156) (width 0.6) (layer "B.Cu") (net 6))
 (segment (start 163.7744 58.852) (end 165.1256 60.2032) (width 0.6) (layer "B.Cu") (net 6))
 (segment (start 127.3812 89.84) (end 127.6098 90.0686) (width 0.6) (layer "B.Cu") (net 6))
 (segment (start 132.8168 63.5105) (end 132.8168 66.7768) (width 0.6) (layer "F.Cu") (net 5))
 (segment (start 147.8536 72.8728) (end 147.8536 75.7176) (width 0.6) (layer "F.Cu") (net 5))
 (segment (start 112.7 86.0808) (end 118.9484 92.3292) (width 0.6) (layer "F.Cu") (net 5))
 (segment (start 112.7 83.0836) (end 112.7 86.0808) (width 0.6) (layer "F.Cu") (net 5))
 (segment (start 132.8168 66.7768) (end 133.02 66.98) (width 0.6) (layer "F.Cu") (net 5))
 (segment (start 147.8536 75.7176) (end 147.9552 75.8192) (width 0.6) (layer "F.Cu") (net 5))
 (via (at 132.8168 63.5105) (size 0.8) (drill 0.4) (layers "F.Cu" "B.Cu") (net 5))
 (via (at 112.7 83.0836) (size 0.8) (drill 0.4) (layers "F.Cu" "B.Cu") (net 5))
 (via (at 118.9484 92.3292) (size 0.8) (drill 0.4) (layers "F.Cu" "B.Cu") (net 5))
 (via (at 147.8536 72.8728) (size 0.8) (drill 0.4) (layers "F.Cu" "B.Cu") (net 5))
 (via (at 147.9552 75.8192) (size 0.8) (drill 0.4) (layers "F.Cu" "B.Cu") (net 5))
 (segment (start 108.6868 92.634) (end 119.2532 92.634) (width 0.6) (layer "B.Cu") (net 5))
 (segment (start 162.2808 61.392) (end 159.3344 61.392) (width 0.6) (layer "B.Cu") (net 5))
 (segment (start 148.7172 85.6744) (end 148.26 86.1316) (width 0.6) (layer "B.Cu") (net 5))
 (segment (start 109.9568 69.6216) (end 108.0868 69.6216) (width 0.6) (layer "B.Cu") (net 5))
 (segment (start 108.0868 69.6216) (end 104.4704 73.238) (width 0.6) (layer "B.Cu") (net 5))
 (segment (start 147.9552 79.3752) (end 148.26 79.68) (width 0.6) (layer "B.Cu") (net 5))
 (segment (start 162.2808 61.392) (end 134.9353 61.392) (width 0.6) (layer "B.Cu") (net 5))
 (segment (start 148.26 79.68) (end 148.26 86.1316) (width 0.6) (layer "B.Cu") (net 5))
 (segment (start 120.6564 94.0372) (end 134.6772 94.0372) (width 0.6) (layer "B.Cu") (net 5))
 (segment (start 131.1761 63.5105) (end 132.8168 63.5105) (width 0.6) (layer "B.Cu") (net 5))
 (segment (start 133.02 66.9292) (end 133.02 66.98) (width 0.6) (layer "B.Cu") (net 5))
 (segment (start 159.3344 61.392) (end 147.8536 72.8728) (width 0.6) (layer "B.Cu") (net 5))
 (segment (start 148.26 86.1316) (end 148.26 87.3) (width 0.6) (layer "B.Cu") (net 5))
 (segment (start 133.02 66.9292) (end 132.8168 66.726) (width 0.6) (layer "B.Cu") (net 5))
 (segment (start 133.02 66.98) (end 133.02 67.1324) (width 0.6) (layer "B.Cu") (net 5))
 (segment (start 134.6772 94.0372) (end 138.1 97.46) (width 0.6) (layer "B.Cu") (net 5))
 (segment (start 149.6824 86.6396) (end 148.7172 85.6744) (width 0.6) (layer "B.Cu") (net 5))
 (segment (start 145.72 89.84) (end 148.26 87.3) (width 0.6) (layer "B.Cu") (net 5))
 (segment (start 145.72 97.46) (end 145.72 89.84) (width 0.6) (layer "B.Cu") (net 5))
 (segment (start 107.6708 83.0836) (end 112.7 83.0836) (width 0.6) (layer "B.Cu") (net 5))
 (segment (start 104.4704 73.238) (end 104.4704 79.8832) (width 0.6) (layer "B.Cu") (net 5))
 (segment (start 134.9353 61.392) (end 132.8168 63.5105) (width 0.6) (layer "B.Cu") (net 5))
 (segment (start 133.02 67.1324) (end 133.66 67.1324) (width 0.6) (layer "B.Cu") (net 5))
 (segment (start 147.9552 75.8192) (end 147.9552 79.3752) (width 0.6) (layer "B.Cu") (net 5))
 (segment (start 160.0964 86.6396) (end 149.6824 86.6396) (width 0.6) (layer "B.Cu") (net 5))
 (segment (start 129.1592 61.4936) (end 131.1761 63.5105) (width 0.6) (layer "B.Cu") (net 5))
 (segment (start 104.4704 79.8832) (end 107.6708 83.0836) (width 0.6) (layer "B.Cu") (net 5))
 (segment (start 118.9484 92.3292) (end 119.2532 92.634) (width 0.6) (layer "B.Cu") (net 5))
 (segment (start 119.2532 92.634) (end 120.6564 94.0372) (width 0.6) (layer "B.Cu") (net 5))
 (segment (start 124.6082 74.092) (end 124.6082 77.78) (width 0.6) (layer "B.Cu") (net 32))
 (segment (start 135.56 65.11) (end 135.26 64.81) (width 0.6) (layer "B.Cu") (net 32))
 (segment (start 125.1316 64.81) (end 124.7716 65.17) (width 0.6) (layer "B.Cu") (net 32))
 (segment (start 124.7048 73.6922) (end 125.1046 74.092) (width 0.6) (layer "B.Cu") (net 32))
 (segment (start 135.26 64.81) (end 125.1316 64.81) (width 0.6) (layer "B.Cu") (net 32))
 (segment (start 124.6082 77.78) (end 124.6888 77.8606) (width 0.6) (layer "B.Cu") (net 32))
 (segment (start 124.7716 65.17) (end 124.7716 67.8436) (width 0.6) (layer "B.Cu") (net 32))
 (segment (start 124.7716 67.8436) (end 124.6082 68.007) (width 0.6) (layer "B.Cu") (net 32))
 (segment (start 124.6082 68.007) (end 124.6082 74.092) (width 0.6) (layer "B.Cu") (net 32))
 (segment (start 135.56 66.98) (end 135.56 65.11) (width 0.6) (layer "B.Cu") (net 32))
 (segment (start 133.02 74.5) (end 133.02 82.86) (width 0.6) (layer "B.Cu") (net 29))
 (segment (start 126.7716 73.8286) (end 126.5082 74.092) (width 0.6) (layer "B.Cu") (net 29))
 (segment (start 133.02 82.86) (end 135.56 85.4) (width 0.6) (layer "B.Cu") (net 29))
 (segment (start 129.0862 76.67) (end 132.7788 76.67) (width 0.6) (layer "B.Cu") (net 29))
 (segment (start 126.5082 74.092) (end 129.0862 76.67) (width 0.6) (layer "B.Cu") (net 29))
 (segment (start 132.7788 76.67) (end 133.02 76.4288) (width 0.6) (layer "B.Cu") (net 29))
 (segment (start 126.7716 67.8436) (end 126.7716 73.8286) (width 0.6) (layer "B.Cu") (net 29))
 (segment (start 133.02 76.4288) (end 133.02 74.5) (width 0.6) (layer "B.Cu") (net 29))
 (segment (start 143.18 84.76) (end 138.1 84.76) (width 0.6) (layer "B.Cu") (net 30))
 (segment (start 135.56 79.04) (end 135.56 77.04) (width 0.6) (layer "B.Cu") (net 30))
 (segment (start 135.56 76.5) (end 135.56 74.5) (width 0.6) (layer "B.Cu") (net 30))
 (segment (start 135.56 74.5) (end 135.56 82.22) (width 0.6) (layer "B.Cu") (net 30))
 (segment (start 138.74 79.68) (end 135.56 76.5) (width 0.6) (layer "B.Cu") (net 30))
 (segment (start 135.56 82.22) (end 138.1 84.76) (width 0.6) (layer "B.Cu") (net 30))
 (segment (start 145.72 79.68) (end 140.64 79.68) (width 0.6) (layer "B.Cu") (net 34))
 (segment (start 152.4 99.36) (end 105.4052 99.36) (width 0.6) (layer "B.Cu") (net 8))
 (segment (start 105.4052 99.36) (end 102.4384 96.3932) (width 0.6) (layer "B.Cu") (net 8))
 (segment (start 102.4384 90.602) (end 102.9464 90.094) (width 0.6) (layer "B.Cu") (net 8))
 (segment (start 102.4384 96.3932) (end 102.4384 90.602) (width 0.6) (layer "B.Cu") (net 8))
 (segment (start 153.34 98.42) (end 152.4 99.36) (width 0.6) (layer "B.Cu") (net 8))
 (segment (start 102.9464 90.094) (end 108.6868 90.094) (width 0.6) (layer "B.Cu") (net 8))
 (segment (start 121.2046 90.348) (end 108.9408 90.348) (width 0.6) (layer "B.Cu") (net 8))
 (segment (start 108.9408 90.348) (end 108.6868 90.094) (width 0.6) (layer "B.Cu") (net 8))
 (segment (start 153.34 97.46) (end 153.34 98.42) (width 0.6) (layer "B.Cu") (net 8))
 (segment (start 141.6052 92.5832) (end 147.3456 92.5832) (width 0.6) (layer "F.Cu") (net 7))
 (segment (start 147.3456 92.5832) (end 147.5488 92.7864) (width 0.6) (layer "F.Cu") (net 7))
 (via (at 141.6052 92.5832) (size 0.8) (drill 0.4) (layers "F.Cu" "B.Cu") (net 7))
 (via (at 147.5488 92.7864) (size 0.8) (drill 0.4) (layers "F.Cu" "B.Cu") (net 7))
 (segment (start 132.328 89.5036) (end 138.5256 89.5036) (width 0.6) (layer "B.Cu") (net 7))
 (segment (start 138.5256 89.5036) (end 141.6052 92.5832) (width 0.6) (layer "B.Cu") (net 7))
 (segment (start 124.6888 79.7606) (end 124.6888 81.8644) (width 0.6) (layer "B.Cu") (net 7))
 (segment (start 150.8 96.0376) (end 147.5488 92.7864) (width 0.6) (layer "B.Cu") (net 7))
 (segment (start 124.6888 85.1476) (end 124.8412 85.3) (width 0.6) (layer "B.Cu") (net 7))
 (segment (start 124.6888 81.8644) (end 132.328 89.5036) (width 0.6) (layer "B.Cu") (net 7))
 (segment (start 124.6888 81.8644) (end 124.6888 85.1476) (width 0.6) (layer "B.Cu") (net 7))
 (segment (start 150.8 97.46) (end 150.8 96.0376) (width 0.6) (layer "B.Cu") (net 7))
 (segment (start 161.9664 81.5596) (end 163.5 83.0932) (width 0.6) (layer "B.Cu") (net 12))
 (segment (start 163.5 83.0932) (end 163.5 97.46) (width 0.6) (layer "B.Cu") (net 12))
 (segment (start 160.0964 81.5596) (end 161.9664 81.5596) (width 0.6) (layer "B.Cu") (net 12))
 (segment (start 162.71 99.21) (end 160.96 97.46) (width 0.6) (layer "B.Cu") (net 11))
 (segment (start 164.3214 99.21) (end 162.71 99.21) (width 0.6) (layer "B.Cu") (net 11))
 (segment (start 160.0964 79.0196) (end 161.9664 79.0196) (width 0.6) (layer "B.Cu") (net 11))
 (segment (start 161.9664 79.0196) (end 167.94 84.9932) (width 0.6) (layer "B.Cu") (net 11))
 (segment (start 167.94 95.5914) (end 164.3214 99.21) (width 0.6) (layer "B.Cu") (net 11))
 (segment (start 167.94 84.9932) (end 167.94 95.5914) (width 0.6) (layer "B.Cu") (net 11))
 (segment (start 160.11 54.558206) (end 161.863794 56.312) (width 0.6) (layer "B.Cu") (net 26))
 (segment (start 160.11 50.05) (end 160.11 54.558206) (width 0.6) (layer "B.Cu") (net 26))
 (segment (start 160.96 49.2) (end 160.11 50.05) (width 0.6) (layer "B.Cu") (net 26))
 (segment (start 161.863794 56.312) (end 162.2808 56.312) (width 0.6) (layer "B.Cu") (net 26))
 (segment (start 162.2808 50.4192) (end 163.5 49.2) (width 0.6) (layer "B.Cu") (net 27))
 (segment (start 162.2808 53.772) (end 162.2808 50.4192) (width 0.6) (layer "B.Cu") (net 27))
 (segment (start 158.42 53.6704) (end 154.8132 57.2772) (width 0.6) (layer "B.Cu") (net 25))
 (segment (start 121.1328 71.806) (end 115.6972 77.2416) (width 0.6) (layer "B.Cu") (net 25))
 (segment (start 158.42 49.2) (end 158.42 53.6704) (width 0.6) (layer "B.Cu") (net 25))
 (segment (start 121.1328 62.3064) (end 121.1328 71.806) (width 0.6) (layer "B.Cu") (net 25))
 (segment (start 115.6972 77.2416) (end 109.9568 77.2416) (width 0.6) (layer "B.Cu") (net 25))
 (segment (start 126.162 57.2772) (end 121.1328 62.3064) (width 0.6) (layer "B.Cu") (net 25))
 (segment (start 154.8132 57.2772) (end 126.162 57.2772) (width 0.6) (layer "B.Cu") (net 25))
 (segment (start 124.5048 55.8356) (end 118.9992 61.3412) (width 0.6) (layer "B.Cu") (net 23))
 (segment (start 153.34 52.6544) (end 153.34 49.2) (width 0.6) (layer "B.Cu") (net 23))
 (segment (start 114.4272 74.7016) (end 109.9568 74.7016) (width 0.6) (layer "B.Cu") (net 23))
 (segment (start 118.9992 70.1296) (end 114.4272 74.7016) (width 0.6) (layer "B.Cu") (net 23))
 (segment (start 149.9172 56.0772) (end 153.1114 52.883) (width 0.6) (layer "B.Cu") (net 23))
 (segment (start 153.1114 52.883) (end 150.1588 55.8356) (width 0.6) (layer "B.Cu") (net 23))
 (segment (start 150.1588 55.8356) (end 124.5048 55.8356) (width 0.6) (layer "B.Cu") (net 23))
 (segment (start 153.1114 52.883) (end 153.34 52.6544) (width 0.6) (layer "B.Cu") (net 23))
 (segment (start 118.9992 61.3412) (end 118.9992 70.1296) (width 0.6) (layer "B.Cu") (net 23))
 (segment (start 112.192 71.7964) (end 111.8268 72.1616) (width 0.6) (layer "B.Cu") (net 22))
 (segment (start 111.8268 72.1616) (end 109.9568 72.1616) (width 0.6) (layer "B.Cu") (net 22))
 (segment (start 145.3644 54.6356) (end 124.007744 54.6356) (width 0.6) (layer "B.Cu") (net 22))
 (segment (start 150.8 49.2) (end 145.3644 54.6356) (width 0.6) (layer "B.Cu") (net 22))
 (segment (start 112.192 66.451344) (end 112.192 71.7964) (width 0.6) (layer "B.Cu") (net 22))
 (segment (start 124.007744 54.6356) (end 112.192 66.451344) (width 0.6) (layer "B.Cu") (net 22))
 (segment (start 121.3992 52.2356) (end 125.9204 52.2356) (width 0.6) (layer "B.Cu") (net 14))
 (segment (start 110.9228 57.7336) (end 115.9012 57.7336) (width 0.6) (layer "B.Cu") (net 14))
 (segment (start 125.9204 52.2356) (end 128.956 49.2) (width 0.6) (layer "B.Cu") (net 14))
 (segment (start 115.9012 57.7336) (end 121.3992 52.2356) (width 0.6) (layer "B.Cu") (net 14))
 (segment (start 113.34 54.6464) (end 113.34 48.3762) (width 0.6) (layer "B.Cu") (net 16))
 (segment (start 112.7928 55.1936) (end 113.34 54.6464) (width 0.6) (layer "B.Cu") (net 16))
 (segment (start 113.34 48.3762) (end 114.4162 47.3) (width 0.6) (layer "B.Cu") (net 16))
 (segment (start 132.136 47.3) (end 134.036 49.2) (width 0.6) (layer "B.Cu") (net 16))
 (segment (start 114.4162 47.3) (end 132.136 47.3) (width 0.6) (layer "B.Cu") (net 16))
 (segment (start 110.9228 55.1936) (end 112.7928 55.1936) (width 0.6) (layer "B.Cu") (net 16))
 (segment (start 132.3404 53.4356) (end 122.4344 53.4356) (width 0.6) (layer "B.Cu") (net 17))
 (segment (start 115.5964 60.2736) (end 110.9228 60.2736) (width 0.6) (layer "B.Cu") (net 17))
 (segment (start 136.576 49.2) (end 132.3404 53.4356) (width 0.6) (layer "B.Cu") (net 17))
 (segment (start 122.4344 53.4356) (end 115.5964 60.2736) (width 0.6) (layer "B.Cu") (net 17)))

